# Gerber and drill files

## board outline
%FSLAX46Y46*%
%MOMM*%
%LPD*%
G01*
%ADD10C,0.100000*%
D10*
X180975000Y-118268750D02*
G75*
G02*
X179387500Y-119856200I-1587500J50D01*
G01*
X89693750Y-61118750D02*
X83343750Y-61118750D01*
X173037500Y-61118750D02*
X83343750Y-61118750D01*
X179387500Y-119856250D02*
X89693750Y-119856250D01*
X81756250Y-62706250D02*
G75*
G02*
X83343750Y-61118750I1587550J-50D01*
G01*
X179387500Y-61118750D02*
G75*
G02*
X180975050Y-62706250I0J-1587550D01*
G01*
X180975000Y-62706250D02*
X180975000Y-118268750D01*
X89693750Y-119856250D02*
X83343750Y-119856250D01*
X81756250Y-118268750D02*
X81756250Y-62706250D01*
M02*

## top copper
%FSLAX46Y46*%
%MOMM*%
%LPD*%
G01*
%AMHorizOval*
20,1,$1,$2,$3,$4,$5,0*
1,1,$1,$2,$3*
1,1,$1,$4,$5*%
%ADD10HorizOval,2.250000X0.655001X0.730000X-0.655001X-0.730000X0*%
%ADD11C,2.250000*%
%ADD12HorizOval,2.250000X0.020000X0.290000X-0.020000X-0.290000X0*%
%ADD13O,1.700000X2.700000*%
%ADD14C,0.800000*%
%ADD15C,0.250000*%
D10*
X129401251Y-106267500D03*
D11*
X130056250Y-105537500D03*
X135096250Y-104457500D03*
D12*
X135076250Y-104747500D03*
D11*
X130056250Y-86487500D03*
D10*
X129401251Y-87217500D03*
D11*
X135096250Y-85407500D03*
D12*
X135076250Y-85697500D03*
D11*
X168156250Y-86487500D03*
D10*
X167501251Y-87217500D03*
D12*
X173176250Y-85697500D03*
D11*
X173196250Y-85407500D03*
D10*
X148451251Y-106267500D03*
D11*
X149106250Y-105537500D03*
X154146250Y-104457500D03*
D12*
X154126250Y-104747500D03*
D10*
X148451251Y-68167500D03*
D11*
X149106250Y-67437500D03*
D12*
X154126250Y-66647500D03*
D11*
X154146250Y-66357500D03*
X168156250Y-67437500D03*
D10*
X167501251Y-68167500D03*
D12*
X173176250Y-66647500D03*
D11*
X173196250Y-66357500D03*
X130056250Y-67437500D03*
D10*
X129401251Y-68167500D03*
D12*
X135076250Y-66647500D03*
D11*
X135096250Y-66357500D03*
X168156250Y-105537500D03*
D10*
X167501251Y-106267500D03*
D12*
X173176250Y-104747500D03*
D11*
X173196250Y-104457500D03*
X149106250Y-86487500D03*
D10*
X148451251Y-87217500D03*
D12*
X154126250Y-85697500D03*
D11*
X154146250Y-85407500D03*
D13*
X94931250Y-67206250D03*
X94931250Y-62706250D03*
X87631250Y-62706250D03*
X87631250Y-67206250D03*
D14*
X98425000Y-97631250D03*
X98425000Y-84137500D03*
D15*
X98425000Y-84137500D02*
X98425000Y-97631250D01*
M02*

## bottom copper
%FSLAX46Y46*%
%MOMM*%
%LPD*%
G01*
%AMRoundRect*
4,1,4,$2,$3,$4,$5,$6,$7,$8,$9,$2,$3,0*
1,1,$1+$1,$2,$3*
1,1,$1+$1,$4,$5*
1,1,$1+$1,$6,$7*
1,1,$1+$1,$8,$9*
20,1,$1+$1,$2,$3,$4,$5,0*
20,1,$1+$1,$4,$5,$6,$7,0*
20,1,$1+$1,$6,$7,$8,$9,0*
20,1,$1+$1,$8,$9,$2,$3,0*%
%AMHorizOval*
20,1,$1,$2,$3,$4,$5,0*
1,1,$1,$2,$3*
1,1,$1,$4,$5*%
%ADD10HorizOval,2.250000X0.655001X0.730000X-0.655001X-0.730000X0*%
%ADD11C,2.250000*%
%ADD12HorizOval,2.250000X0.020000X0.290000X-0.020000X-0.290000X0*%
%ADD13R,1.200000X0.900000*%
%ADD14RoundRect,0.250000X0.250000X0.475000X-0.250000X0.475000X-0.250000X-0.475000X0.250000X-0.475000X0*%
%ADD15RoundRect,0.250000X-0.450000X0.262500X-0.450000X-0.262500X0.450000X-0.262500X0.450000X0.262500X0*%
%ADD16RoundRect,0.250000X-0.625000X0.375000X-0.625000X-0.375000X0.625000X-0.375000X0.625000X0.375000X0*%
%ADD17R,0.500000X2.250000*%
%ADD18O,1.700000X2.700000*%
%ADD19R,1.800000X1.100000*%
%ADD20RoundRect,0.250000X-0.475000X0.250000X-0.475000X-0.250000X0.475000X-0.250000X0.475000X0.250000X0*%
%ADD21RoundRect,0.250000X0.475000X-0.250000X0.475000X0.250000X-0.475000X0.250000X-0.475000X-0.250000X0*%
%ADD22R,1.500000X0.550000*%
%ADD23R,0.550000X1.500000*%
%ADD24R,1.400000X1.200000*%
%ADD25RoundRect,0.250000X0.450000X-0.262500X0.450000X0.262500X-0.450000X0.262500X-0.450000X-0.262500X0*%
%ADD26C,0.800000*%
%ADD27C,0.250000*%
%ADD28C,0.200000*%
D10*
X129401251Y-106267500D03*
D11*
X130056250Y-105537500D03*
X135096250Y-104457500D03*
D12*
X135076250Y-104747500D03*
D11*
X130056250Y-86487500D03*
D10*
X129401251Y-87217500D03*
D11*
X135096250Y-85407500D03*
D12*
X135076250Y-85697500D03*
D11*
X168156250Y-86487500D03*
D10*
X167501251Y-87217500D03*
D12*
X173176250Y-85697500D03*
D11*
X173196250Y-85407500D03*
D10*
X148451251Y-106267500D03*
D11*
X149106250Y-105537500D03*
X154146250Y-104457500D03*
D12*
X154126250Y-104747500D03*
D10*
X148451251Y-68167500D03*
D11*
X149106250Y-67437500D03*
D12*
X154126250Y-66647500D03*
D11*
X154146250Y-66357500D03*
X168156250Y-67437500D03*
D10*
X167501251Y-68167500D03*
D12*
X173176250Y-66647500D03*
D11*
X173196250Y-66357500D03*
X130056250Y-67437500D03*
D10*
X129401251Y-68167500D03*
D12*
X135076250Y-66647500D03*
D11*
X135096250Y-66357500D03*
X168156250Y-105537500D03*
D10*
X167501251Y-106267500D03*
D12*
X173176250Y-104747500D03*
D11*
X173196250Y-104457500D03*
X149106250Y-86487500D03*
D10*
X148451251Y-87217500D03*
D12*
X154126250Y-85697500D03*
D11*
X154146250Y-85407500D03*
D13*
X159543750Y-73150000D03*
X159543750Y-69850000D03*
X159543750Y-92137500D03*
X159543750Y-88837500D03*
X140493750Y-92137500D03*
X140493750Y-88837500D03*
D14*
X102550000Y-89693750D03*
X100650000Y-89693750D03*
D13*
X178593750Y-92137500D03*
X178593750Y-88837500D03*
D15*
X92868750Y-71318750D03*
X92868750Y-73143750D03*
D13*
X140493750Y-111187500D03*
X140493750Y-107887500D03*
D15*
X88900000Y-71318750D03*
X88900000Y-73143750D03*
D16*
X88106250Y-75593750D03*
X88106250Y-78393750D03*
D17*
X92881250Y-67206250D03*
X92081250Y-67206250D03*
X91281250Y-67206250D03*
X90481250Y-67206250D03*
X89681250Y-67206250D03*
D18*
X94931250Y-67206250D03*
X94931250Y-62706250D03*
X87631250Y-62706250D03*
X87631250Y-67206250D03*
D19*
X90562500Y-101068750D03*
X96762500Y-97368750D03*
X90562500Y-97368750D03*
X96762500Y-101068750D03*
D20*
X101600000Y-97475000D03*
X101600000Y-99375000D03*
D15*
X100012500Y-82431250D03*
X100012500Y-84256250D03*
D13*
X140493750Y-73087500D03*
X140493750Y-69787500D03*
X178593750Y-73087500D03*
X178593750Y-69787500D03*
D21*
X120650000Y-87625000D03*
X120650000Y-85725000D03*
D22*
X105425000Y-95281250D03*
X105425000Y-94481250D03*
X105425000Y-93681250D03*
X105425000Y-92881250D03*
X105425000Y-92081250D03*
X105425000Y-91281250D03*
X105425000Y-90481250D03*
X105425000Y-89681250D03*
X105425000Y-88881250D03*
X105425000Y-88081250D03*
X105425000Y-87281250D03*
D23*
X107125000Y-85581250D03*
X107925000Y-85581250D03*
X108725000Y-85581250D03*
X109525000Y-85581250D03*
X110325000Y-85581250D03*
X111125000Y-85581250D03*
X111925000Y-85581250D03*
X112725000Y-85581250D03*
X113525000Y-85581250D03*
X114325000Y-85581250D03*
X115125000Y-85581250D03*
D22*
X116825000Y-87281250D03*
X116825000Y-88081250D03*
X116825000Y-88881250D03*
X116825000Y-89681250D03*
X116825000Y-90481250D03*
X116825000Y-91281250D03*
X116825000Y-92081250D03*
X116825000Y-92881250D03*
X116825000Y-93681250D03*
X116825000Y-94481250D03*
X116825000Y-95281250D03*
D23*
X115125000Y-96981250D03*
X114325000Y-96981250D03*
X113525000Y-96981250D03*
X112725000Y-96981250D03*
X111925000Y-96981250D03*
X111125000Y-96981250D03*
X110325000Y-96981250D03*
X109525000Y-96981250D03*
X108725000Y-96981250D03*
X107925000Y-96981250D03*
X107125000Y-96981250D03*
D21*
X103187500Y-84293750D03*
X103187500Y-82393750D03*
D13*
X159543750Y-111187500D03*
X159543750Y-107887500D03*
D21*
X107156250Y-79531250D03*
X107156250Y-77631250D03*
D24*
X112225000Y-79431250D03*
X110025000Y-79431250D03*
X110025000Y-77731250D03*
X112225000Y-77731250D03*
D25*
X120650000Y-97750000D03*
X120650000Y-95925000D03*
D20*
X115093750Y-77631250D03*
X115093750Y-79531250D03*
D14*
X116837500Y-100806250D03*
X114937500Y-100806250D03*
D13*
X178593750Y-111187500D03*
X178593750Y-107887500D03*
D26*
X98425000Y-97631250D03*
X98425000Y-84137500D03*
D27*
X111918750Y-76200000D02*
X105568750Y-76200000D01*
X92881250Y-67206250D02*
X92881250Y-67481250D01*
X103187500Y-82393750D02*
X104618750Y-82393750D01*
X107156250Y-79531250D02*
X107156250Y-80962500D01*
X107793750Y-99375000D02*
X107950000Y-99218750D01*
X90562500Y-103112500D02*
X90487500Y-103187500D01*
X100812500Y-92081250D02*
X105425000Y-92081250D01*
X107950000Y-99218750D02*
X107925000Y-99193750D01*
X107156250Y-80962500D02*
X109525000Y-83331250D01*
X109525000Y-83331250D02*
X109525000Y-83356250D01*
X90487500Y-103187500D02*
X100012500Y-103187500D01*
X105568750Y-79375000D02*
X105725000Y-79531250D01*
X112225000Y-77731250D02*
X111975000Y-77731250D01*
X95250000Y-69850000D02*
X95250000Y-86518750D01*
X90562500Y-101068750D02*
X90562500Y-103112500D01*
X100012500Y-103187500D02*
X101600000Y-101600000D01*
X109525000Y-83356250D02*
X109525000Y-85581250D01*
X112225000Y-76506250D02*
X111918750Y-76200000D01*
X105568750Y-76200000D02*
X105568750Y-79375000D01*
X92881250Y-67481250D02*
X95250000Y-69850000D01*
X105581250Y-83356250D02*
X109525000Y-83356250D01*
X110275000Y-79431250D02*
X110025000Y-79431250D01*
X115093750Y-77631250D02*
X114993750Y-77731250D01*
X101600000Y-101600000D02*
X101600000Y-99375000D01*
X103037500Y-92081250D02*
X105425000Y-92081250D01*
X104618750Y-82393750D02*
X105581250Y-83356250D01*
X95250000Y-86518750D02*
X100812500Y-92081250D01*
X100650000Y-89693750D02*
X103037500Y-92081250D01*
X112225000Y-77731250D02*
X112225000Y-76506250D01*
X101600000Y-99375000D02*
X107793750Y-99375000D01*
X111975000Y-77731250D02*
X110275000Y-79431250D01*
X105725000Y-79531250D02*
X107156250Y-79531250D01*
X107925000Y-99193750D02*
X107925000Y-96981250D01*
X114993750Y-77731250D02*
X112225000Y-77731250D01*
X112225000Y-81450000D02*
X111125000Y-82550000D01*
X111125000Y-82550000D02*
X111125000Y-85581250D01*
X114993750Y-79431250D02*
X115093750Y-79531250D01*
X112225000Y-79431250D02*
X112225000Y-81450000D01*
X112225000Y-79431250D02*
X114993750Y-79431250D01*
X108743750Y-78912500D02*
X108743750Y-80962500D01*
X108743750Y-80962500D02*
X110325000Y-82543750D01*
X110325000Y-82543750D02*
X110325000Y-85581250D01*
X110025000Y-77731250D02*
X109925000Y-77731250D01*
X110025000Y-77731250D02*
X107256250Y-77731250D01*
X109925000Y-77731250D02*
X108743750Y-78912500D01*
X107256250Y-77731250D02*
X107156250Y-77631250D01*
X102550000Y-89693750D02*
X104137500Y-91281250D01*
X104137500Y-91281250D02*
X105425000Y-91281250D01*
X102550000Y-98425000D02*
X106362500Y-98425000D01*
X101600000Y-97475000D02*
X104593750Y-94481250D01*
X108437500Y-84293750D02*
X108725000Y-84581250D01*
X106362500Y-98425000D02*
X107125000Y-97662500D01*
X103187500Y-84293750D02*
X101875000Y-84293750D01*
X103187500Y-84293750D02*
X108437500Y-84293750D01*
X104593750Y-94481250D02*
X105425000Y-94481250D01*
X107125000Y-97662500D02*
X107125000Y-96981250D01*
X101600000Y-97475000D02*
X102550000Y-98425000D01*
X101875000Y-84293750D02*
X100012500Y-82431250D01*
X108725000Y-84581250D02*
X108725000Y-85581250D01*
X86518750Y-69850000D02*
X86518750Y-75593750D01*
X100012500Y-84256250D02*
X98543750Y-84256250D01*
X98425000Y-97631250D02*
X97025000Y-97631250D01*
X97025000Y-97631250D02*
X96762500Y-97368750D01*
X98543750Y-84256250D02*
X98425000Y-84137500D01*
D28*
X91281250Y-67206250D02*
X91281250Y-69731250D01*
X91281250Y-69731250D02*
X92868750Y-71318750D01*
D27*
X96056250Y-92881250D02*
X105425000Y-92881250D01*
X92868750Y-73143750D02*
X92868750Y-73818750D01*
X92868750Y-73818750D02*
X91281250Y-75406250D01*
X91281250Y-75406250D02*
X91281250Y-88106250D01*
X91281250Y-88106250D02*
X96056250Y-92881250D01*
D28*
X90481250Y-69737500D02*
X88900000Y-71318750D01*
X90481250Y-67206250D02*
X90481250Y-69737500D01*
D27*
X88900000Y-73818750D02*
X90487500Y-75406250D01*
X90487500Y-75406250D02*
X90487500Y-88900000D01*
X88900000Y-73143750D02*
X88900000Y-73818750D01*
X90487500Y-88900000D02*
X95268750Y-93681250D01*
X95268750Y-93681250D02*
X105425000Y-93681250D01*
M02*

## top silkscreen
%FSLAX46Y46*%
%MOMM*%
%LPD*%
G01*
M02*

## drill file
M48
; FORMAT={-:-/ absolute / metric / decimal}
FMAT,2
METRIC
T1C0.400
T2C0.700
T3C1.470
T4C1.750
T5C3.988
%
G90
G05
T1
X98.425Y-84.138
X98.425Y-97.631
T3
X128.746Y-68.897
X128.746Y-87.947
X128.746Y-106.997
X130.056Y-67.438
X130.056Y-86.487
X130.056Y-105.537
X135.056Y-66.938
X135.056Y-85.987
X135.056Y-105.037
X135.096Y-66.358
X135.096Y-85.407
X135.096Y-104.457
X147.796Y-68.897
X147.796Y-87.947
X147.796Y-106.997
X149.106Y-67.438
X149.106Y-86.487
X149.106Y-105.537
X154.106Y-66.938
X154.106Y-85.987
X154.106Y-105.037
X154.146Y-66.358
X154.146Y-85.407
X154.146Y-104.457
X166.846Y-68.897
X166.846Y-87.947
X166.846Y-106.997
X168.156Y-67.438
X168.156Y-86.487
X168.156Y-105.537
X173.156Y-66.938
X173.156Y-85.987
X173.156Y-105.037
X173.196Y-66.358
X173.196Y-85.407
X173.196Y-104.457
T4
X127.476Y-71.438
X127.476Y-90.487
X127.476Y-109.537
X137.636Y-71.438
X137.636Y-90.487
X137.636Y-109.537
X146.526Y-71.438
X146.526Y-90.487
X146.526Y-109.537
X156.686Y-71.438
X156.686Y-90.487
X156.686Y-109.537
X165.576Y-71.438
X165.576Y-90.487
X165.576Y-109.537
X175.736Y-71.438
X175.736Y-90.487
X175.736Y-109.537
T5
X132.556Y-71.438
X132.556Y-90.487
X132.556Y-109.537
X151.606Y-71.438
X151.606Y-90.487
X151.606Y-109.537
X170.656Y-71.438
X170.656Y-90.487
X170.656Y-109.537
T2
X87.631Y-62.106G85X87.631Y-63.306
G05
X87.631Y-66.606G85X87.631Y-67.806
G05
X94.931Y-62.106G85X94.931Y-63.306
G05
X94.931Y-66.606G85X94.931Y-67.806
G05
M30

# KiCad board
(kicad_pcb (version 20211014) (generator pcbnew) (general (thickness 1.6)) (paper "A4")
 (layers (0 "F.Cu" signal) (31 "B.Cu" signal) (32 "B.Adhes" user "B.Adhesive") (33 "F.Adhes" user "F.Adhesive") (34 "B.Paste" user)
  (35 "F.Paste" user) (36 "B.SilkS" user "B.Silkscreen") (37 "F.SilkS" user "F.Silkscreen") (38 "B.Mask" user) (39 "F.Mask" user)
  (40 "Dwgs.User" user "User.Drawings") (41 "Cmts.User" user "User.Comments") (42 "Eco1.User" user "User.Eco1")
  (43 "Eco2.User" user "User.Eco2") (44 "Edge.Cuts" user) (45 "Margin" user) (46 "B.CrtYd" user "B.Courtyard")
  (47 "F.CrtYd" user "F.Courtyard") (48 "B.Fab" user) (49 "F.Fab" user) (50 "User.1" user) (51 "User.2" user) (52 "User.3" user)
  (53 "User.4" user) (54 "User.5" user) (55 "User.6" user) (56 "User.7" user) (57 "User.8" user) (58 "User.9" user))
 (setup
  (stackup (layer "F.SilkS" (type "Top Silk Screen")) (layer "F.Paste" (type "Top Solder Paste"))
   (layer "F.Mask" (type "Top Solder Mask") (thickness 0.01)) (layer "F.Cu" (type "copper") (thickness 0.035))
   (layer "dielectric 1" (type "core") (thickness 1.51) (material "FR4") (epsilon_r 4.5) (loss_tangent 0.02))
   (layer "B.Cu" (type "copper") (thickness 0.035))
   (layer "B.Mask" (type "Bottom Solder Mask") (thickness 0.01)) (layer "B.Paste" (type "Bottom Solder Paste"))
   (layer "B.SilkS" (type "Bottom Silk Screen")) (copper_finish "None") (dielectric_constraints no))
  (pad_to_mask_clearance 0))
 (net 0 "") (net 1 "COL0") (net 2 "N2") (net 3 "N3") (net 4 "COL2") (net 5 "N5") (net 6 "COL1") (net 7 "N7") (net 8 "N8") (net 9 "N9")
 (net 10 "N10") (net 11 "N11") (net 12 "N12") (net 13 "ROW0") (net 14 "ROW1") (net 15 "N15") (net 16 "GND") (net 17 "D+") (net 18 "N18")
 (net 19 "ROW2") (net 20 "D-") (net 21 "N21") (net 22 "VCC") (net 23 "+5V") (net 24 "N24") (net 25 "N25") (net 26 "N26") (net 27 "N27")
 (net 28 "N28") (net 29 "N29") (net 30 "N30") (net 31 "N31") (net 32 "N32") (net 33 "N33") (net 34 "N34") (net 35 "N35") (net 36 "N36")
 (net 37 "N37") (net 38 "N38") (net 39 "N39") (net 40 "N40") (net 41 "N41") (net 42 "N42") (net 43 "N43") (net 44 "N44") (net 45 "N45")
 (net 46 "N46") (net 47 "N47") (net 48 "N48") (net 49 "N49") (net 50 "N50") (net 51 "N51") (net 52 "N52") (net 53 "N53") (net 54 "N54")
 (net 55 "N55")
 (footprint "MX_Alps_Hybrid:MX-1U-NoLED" (layer "F.Cu") (at 132.55625 109.5375)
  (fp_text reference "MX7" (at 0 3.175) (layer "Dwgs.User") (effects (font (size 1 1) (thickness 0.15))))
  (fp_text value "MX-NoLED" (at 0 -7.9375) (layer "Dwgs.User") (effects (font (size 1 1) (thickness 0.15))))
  (pad "" np_thru_hole circle locked (at -5.08 0 48.0996) (size 1.75 1.75) (drill 1.75) (layers *.Cu *.Mask))
  (pad "" np_thru_hole circle locked (at 5.08 0 48.0996) (size 1.75 1.75) (drill 1.75) (layers *.Cu *.Mask))
  (pad "" np_thru_hole circle locked (at 0 0) (size 3.9878 3.9878) (drill 3.9878) (layers *.Cu *.Mask))
  (pad "1" thru_hole oval locked (at -3.81 -2.54 48.0996) (size 4.211556 2.25) (drill 1.47 (offset 0.980778 0)) (layers *.Cu "B.Mask")
   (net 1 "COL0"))
  (pad "1" thru_hole circle locked (at -2.5 -4) (size 2.25 2.25) (drill 1.47) (layers *.Cu "B.Mask") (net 1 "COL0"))
  (pad "2" thru_hole circle locked (at 2.54 -5.08) (size 2.25 2.25) (drill 1.47) (layers *.Cu "B.Mask") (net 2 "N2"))
  (pad "2" thru_hole oval locked (at 2.5 -4.5 86.0548) (size 2.831378 2.25) (drill 1.47 (offset 0.290689 0)) (layers *.Cu "B.Mask")
   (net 2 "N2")))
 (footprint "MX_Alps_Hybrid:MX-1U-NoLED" (layer "F.Cu") (at 132.55625 90.4875)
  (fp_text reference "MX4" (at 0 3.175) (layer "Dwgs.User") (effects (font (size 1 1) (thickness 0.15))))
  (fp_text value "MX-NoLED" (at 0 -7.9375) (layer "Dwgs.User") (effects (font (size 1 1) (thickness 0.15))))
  (pad "" np_thru_hole circle locked (at 0 0) (size 3.9878 3.9878) (drill 3.9878) (layers *.Cu *.Mask))
  (pad "" np_thru_hole circle locked (at 5.08 0 48.0996) (size 1.75 1.75) (drill 1.75) (layers *.Cu *.Mask))
  (pad "" np_thru_hole circle locked (at -5.08 0 48.0996) (size 1.75 1.75) (drill 1.75) (layers *.Cu *.Mask))
  (pad "1" thru_hole circle locked (at -2.5 -4) (size 2.25 2.25) (drill 1.47) (layers *.Cu "B.Mask") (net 1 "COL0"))
  (pad "1" thru_hole oval locked (at -3.81 -2.54 48.0996) (size 4.211556 2.25) (drill 1.47 (offset 0.980778 0)) (layers *.Cu "B.Mask")
   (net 1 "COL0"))
  (pad "2" thru_hole circle locked (at 2.54 -5.08) (size 2.25 2.25) (drill 1.47) (layers *.Cu "B.Mask") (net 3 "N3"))
  (pad "2" thru_hole oval locked (at 2.5 -4.5 86.0548) (size 2.831378 2.25) (drill 1.47 (offset 0.290689 0)) (layers *.Cu "B.Mask")
   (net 3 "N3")))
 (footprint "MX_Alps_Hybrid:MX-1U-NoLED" (layer "F.Cu") (at 170.65625 90.4875)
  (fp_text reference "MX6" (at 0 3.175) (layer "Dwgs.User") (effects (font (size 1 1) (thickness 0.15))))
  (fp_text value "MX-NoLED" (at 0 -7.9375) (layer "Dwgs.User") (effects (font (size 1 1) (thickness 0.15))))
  (pad "" np_thru_hole circle locked (at -5.08 0 48.0996) (size 1.75 1.75) (drill 1.75) (layers *.Cu *.Mask))
  (pad "" np_thru_hole circle locked (at 5.08 0 48.0996) (size 1.75 1.75) (drill 1.75) (layers *.Cu *.Mask))
  (pad "" np_thru_hole circle locked (at 0 0) (size 3.9878 3.9878) (drill 3.9878) (layers *.Cu *.Mask))
  (pad "1" thru_hole circle locked (at -2.5 -4) (size 2.25 2.25) (drill 1.47) (layers *.Cu "B.Mask") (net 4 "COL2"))
  (pad "1" thru_hole oval locked (at -3.81 -2.54 48.0996) (size 4.211556 2.25) (drill 1.47 (offset 0.980778 0)) (layers *.Cu "B.Mask")
   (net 4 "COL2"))
  (pad "2" thru_hole oval locked (at 2.5 -4.5 86.0548) (size 2.831378 2.25) (drill 1.47 (offset 0.290689 0)) (layers *.Cu "B.Mask")
   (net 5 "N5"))
  (pad "2" thru_hole circle locked (at 2.54 -5.08) (size 2.25 2.25) (drill 1.47) (layers *.Cu "B.Mask") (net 5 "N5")))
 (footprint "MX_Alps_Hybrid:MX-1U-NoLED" (layer "F.Cu") (at 151.60625 109.5375)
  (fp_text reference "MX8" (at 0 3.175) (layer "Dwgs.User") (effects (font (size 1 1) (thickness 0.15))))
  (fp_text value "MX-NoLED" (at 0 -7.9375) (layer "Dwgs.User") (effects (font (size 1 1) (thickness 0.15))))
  (pad "" np_thru_hole circle locked (at -5.08 0 48.0996) (size 1.75 1.75) (drill 1.75) (layers *.Cu *.Mask))
  (pad "" np_thru_hole circle locked (at 0 0) (size 3.9878 3.9878) (drill 3.9878) (layers *.Cu *.Mask))
  (pad "" np_thru_hole circle locked (at 5.08 0 48.0996) (size 1.75 1.75) (drill 1.75) (layers *.Cu *.Mask))
  (pad "1" thru_hole oval locked (at -3.81 -2.54 48.0996) (size 4.211556 2.25) (drill 1.47 (offset 0.980778 0)) (layers *.Cu "B.Mask")
   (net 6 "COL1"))
  (pad "1" thru_hole circle locked (at -2.5 -4) (size 2.25 2.25) (drill 1.47) (layers *.Cu "B.Mask") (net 6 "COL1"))
  (pad "2" thru_hole circle locked (at 2.54 -5.08) (size 2.25 2.25) (drill 1.47) (layers *.Cu "B.Mask") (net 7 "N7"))
  (pad "2" thru_hole oval locked (at 2.5 -4.5 86.0548) (size 2.831378 2.25) (drill 1.47 (offset 0.290689 0)) (layers *.Cu "B.Mask")
   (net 7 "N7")))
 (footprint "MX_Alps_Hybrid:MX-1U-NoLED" (layer "F.Cu") (at 151.60625 71.4375)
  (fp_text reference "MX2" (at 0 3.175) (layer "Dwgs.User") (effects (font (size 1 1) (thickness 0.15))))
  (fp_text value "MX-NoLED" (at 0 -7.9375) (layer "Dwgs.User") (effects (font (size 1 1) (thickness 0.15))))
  (pad "" np_thru_hole circle locked (at 5.08 0 48.0996) (size 1.75 1.75) (drill 1.75) (layers *.Cu *.Mask))
  (pad "" np_thru_hole circle locked (at -5.08 0 48.0996) (size 1.75 1.75) (drill 1.75) (layers *.Cu *.Mask))
  (pad "" np_thru_hole circle locked (at 0 0) (size 3.9878 3.9878) (drill 3.9878) (layers *.Cu *.Mask))
  (pad "1" thru_hole oval locked (at -3.81 -2.54 48.0996) (size 4.211556 2.25) (drill 1.47 (offset 0.980778 0)) (layers *.Cu "B.Mask")
   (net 6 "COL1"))
  (pad "1" thru_hole circle locked (at -2.5 -4) (size 2.25 2.25) (drill 1.47) (layers *.Cu "B.Mask") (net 6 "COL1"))
  (pad "2" thru_hole oval locked (at 2.5 -4.5 86.0548) (size 2.831378 2.25) (drill 1.47 (offset 0.290689 0)) (layers *.Cu "B.Mask")
   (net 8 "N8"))
  (pad "2" thru_hole circle locked (at 2.54 -5.08) (size 2.25 2.25) (drill 1.47) (layers *.Cu "B.Mask") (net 8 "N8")))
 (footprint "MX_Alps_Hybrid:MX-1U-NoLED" (layer "F.Cu") (at 170.65625 71.4375)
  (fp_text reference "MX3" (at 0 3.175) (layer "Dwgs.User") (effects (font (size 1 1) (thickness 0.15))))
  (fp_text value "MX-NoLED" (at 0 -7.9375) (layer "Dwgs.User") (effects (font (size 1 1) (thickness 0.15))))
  (pad "" np_thru_hole circle locked (at -5.08 0 48.0996) (size 1.75 1.75) (drill 1.75) (layers *.Cu *.Mask))
  (pad "" np_thru_hole circle locked (at 5.08 0 48.0996) (size 1.75 1.75) (drill 1.75) (layers *.Cu *.Mask))
  (pad "" np_thru_hole circle locked (at 0 0) (size 3.9878 3.9878) (drill 3.9878) (layers *.Cu *.Mask))
  (pad "1" thru_hole circle locked (at -2.5 -4) (size 2.25 2.25) (drill 1.47) (layers *.Cu "B.Mask") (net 4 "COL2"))
  (pad "1" thru_hole oval locked (at -3.81 -2.54 48.0996) (size 4.211556 2.25) (drill 1.47 (offset 0.980778 0)) (layers *.Cu "B.Mask")
   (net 4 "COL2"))
  (pad "2" thru_hole oval locked (at 2.5 -4.5 86.0548) (size 2.831378 2.25) (drill 1.47 (offset 0.290689 0)) (layers *.Cu "B.Mask")
   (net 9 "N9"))
  (pad "2" thru_hole circle locked (at 2.54 -5.08) (size 2.25 2.25) (drill 1.47) (layers *.Cu "B.Mask") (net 9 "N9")))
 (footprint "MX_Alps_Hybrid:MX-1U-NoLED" (layer "F.Cu") (at 132.55625 71.4375)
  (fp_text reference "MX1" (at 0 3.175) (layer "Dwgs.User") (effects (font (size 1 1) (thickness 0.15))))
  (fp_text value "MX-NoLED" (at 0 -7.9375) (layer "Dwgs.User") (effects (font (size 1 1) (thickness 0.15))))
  (pad "" np_thru_hole circle locked (at 5.08 0 48.0996) (size 1.75 1.75) (drill 1.75) (layers *.Cu *.Mask))
  (pad "" np_thru_hole circle locked (at -5.08 0 48.0996) (size 1.75 1.75) (drill 1.75) (layers *.Cu *.Mask))
  (pad "" np_thru_hole circle locked (at 0 0) (size 3.9878 3.9878) (drill 3.9878) (layers *.Cu *.Mask))
  (pad "1" thru_hole circle locked (at -2.5 -4) (size 2.25 2.25) (drill 1.47) (layers *.Cu "B.Mask") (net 1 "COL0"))
  (pad "1" thru_hole oval locked (at -3.81 -2.54 48.0996) (size 4.211556 2.25) (drill 1.47 (offset 0.980778 0)) (layers *.Cu "B.Mask")
   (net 1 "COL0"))
  (pad "2" thru_hole oval locked (at 2.5 -4.5 86.0548) (size 2.831378 2.25) (drill 1.47 (offset 0.290689 0)) (layers *.Cu "B.Mask")
   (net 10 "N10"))
  (pad "2" thru_hole circle locked (at 2.54 -5.08) (size 2.25 2.25) (drill 1.47) (layers *.Cu "B.Mask") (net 10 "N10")))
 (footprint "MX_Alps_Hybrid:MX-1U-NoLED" (layer "F.Cu") (at 170.65625 109.5375)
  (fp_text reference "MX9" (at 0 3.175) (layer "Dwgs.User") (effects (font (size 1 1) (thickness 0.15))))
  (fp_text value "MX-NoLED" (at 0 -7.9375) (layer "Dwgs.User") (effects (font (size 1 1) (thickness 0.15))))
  (pad "" np_thru_hole circle locked (at -5.08 0 48.0996) (size 1.75 1.75) (drill 1.75) (layers *.Cu *.Mask))
  (pad "" np_thru_hole circle locked (at 0 0) (size 3.9878 3.9878) (drill 3.9878) (layers *.Cu *.Mask))
  (pad "" np_thru_hole circle locked (at 5.08 0 48.0996) (size 1.75 1.75) (drill 1.75) (layers *.Cu *.Mask))
  (pad "1" thru_hole circle locked (at -2.5 -4) (size 2.25 2.25) (drill 1.47) (layers *.Cu "B.Mask") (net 4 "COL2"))
  (pad "1" thru_hole oval locked (at -3.81 -2.54 48.0996) (size 4.211556 2.25) (drill 1.47 (offset 0.980778 0)) (layers *.Cu "B.Mask")
   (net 4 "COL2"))
  (pad "2" thru_hole oval locked (at 2.5 -4.5 86.0548) (size 2.831378 2.25) (drill 1.47 (offset 0.290689 0)) (layers *.Cu "B.Mask")
   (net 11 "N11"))
  (pad "2" thru_hole circle locked (at 2.54 -5.08) (size 2.25 2.25) (drill 1.47) (layers *.Cu "B.Mask") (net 11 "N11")))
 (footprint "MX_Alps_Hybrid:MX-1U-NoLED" (layer "F.Cu") (at 151.60625 90.4875)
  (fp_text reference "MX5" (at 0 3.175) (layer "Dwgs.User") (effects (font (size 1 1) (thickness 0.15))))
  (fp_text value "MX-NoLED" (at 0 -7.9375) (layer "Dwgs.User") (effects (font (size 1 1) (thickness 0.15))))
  (pad "" np_thru_hole circle locked (at 5.08 0 48.0996) (size 1.75 1.75) (drill 1.75) (layers *.Cu *.Mask))
  (pad "" np_thru_hole circle locked (at -5.08 0 48.0996) (size 1.75 1.75) (drill 1.75) (layers *.Cu *.Mask))
  (pad "" np_thru_hole circle locked (at 0 0) (size 3.9878 3.9878) (drill 3.9878) (layers *.Cu *.Mask))
  (pad "1" thru_hole circle locked (at -2.5 -4) (size 2.25 2.25) (drill 1.47) (layers *.Cu "B.Mask") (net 6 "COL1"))
  (pad "1" thru_hole oval locked (at -3.81 -2.54 48.0996) (size 4.211556 2.25) (drill 1.47 (offset 0.980778 0)) (layers *.Cu "B.Mask")
   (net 6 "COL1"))
  (pad "2" thru_hole oval locked (at 2.5 -4.5 86.0548) (size 2.831378 2.25) (drill 1.47 (offset 0.290689 0)) (layers *.Cu "B.Mask")
   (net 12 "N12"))
  (pad "2" thru_hole circle locked (at 2.54 -5.08) (size 2.25 2.25) (drill 1.47) (layers *.Cu "B.Mask") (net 12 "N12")))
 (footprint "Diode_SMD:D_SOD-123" (layer "B.Cu") (at 159.54375 71.5 90)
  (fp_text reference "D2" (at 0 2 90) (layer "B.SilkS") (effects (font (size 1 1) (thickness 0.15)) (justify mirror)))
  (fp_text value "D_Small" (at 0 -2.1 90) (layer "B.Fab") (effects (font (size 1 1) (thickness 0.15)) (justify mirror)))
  (pad "1" smd rect (at -1.65 0 90) (size 0.9 1.2) (layers "B.Cu" "B.Paste" "B.Mask") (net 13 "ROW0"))
  (pad "2" smd rect (at 1.65 0 90) (size 0.9 1.2) (layers "B.Cu" "B.Paste" "B.Mask") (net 8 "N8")))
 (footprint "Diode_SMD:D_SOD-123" (layer "B.Cu") (at 159.54375 90.4875 90)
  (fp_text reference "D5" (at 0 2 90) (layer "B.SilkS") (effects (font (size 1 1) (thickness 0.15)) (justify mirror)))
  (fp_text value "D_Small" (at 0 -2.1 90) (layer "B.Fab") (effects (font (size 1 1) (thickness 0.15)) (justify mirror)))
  (pad "1" smd rect (at -1.65 0 90) (size 0.9 1.2) (layers "B.Cu" "B.Paste" "B.Mask") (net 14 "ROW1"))
  (pad "2" smd rect (at 1.65 0 90) (size 0.9 1.2) (layers "B.Cu" "B.Paste" "B.Mask") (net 12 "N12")))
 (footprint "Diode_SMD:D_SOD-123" (layer "B.Cu") (at 140.49375 90.4875 90)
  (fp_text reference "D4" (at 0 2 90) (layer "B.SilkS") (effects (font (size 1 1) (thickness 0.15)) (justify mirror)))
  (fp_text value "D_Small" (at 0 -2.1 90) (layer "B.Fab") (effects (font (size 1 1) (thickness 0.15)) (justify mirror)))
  (pad "1" smd rect (at -1.65 0 90) (size 0.9 1.2) (layers "B.Cu" "B.Paste" "B.Mask") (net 14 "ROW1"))
  (pad "2" smd rect (at 1.65 0 90) (size 0.9 1.2) (layers "B.Cu" "B.Paste" "B.Mask") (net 3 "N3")))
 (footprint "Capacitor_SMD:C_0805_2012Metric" (layer "B.Cu") (at 101.6 89.69375 180)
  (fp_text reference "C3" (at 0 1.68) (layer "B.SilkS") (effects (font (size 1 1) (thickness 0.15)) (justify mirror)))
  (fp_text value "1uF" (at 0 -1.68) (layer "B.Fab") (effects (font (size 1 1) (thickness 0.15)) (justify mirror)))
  (pad "1" smd roundrect (at -0.95 0 180) (size 1 1.45) (layers "B.Cu" "B.Paste" "B.Mask") (roundrect_rratio 0.25) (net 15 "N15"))
  (pad "2" smd roundrect (at 0.95 0 180) (size 1 1.45) (layers "B.Cu" "B.Paste" "B.Mask") (roundrect_rratio 0.25) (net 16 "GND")))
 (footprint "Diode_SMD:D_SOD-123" (layer "B.Cu") (at 178.59375 90.4875 90)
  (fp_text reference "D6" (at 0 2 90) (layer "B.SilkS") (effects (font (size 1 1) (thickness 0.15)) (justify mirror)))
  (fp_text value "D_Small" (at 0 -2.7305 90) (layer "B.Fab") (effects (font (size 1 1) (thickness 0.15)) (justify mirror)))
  (pad "1" smd rect (at -1.65 0 90) (size 0.9 1.2) (layers "B.Cu" "B.Paste" "B.Mask") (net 14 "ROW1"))
  (pad "2" smd rect (at 1.65 0 90) (size 0.9 1.2) (layers "B.Cu" "B.Paste" "B.Mask") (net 5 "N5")))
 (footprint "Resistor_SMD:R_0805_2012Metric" (layer "B.Cu") (at 92.86875 72.23125 -90)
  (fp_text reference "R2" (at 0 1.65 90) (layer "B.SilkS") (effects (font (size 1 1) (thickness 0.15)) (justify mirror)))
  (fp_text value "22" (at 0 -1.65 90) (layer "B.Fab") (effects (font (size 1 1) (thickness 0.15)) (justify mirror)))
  (pad "1" smd roundrect (at -0.9125 0 270) (size 1.025 1.4) (layers "B.Cu" "B.Paste" "B.Mask") (roundrect_rratio 0.243902) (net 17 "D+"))
  (pad "2" smd roundrect (at 0.9125 0 270) (size 1.025 1.4) (layers "B.Cu" "B.Paste" "B.Mask") (roundrect_rratio 0.243902) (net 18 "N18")))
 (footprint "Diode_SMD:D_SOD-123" (layer "B.Cu") (at 140.49375 109.5375 90)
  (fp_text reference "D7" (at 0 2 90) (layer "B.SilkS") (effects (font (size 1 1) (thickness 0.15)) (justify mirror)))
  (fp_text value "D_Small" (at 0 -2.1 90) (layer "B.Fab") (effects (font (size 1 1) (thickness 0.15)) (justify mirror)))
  (pad "1" smd rect (at -1.65 0 90) (size 0.9 1.2) (layers "B.Cu" "B.Paste" "B.Mask") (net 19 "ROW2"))
  (pad "2" smd rect (at 1.65 0 90) (size 0.9 1.2) (layers "B.Cu" "B.Paste" "B.Mask") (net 2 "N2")))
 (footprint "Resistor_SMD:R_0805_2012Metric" (layer "B.Cu") (at 88.9 72.23125 -90)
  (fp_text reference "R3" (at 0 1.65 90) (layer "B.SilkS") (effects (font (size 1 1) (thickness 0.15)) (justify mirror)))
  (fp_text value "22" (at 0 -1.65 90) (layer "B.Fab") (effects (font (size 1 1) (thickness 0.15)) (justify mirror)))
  (pad "1" smd roundrect (at -0.9125 0 270) (size 1.025 1.4) (layers "B.Cu" "B.Paste" "B.Mask") (roundrect_rratio 0.243902) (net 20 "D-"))
  (pad "2" smd roundrect (at 0.9125 0 270) (size 1.025 1.4) (layers "B.Cu" "B.Paste" "B.Mask") (roundrect_rratio 0.243902) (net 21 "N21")))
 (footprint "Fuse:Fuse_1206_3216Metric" (layer "B.Cu") (at 88.10625 76.99375 -90)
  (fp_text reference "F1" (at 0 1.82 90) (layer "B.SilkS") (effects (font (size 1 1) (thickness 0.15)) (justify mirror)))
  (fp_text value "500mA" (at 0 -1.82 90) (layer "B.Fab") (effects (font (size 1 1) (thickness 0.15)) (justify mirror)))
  (pad "1" smd roundrect (at -1.4 0 270) (size 1.25 1.75) (layers "B.Cu" "B.Paste" "B.Mask") (roundrect_rratio 0.2) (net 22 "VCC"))
  (pad "2" smd roundrect (at 1.4 0 270) (size 1.25 1.75) (layers "B.Cu" "B.Paste" "B.Mask") (roundrect_rratio 0.2) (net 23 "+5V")))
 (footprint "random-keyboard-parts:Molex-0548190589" (layer "B.Cu") (at 91.28125 62.70625 -90)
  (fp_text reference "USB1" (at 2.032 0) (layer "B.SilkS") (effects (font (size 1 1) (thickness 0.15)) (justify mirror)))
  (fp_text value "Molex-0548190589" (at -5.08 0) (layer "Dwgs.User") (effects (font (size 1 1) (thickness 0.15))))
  (pad "1" smd rect locked (at 4.5 -1.6 270) (size 2.25 0.5) (layers "B.Cu" "B.Paste" "B.Mask") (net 16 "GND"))
  (pad "2" smd rect locked (at 4.5 -0.8 270) (size 2.25 0.5) (layers "B.Cu" "B.Paste" "B.Mask") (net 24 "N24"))
  (pad "3" smd rect locked (at 4.5 0 270) (size 2.25 0.5) (layers "B.Cu" "B.Paste" "B.Mask") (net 17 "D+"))
  (pad "4" smd rect locked (at 4.5 0.8 270) (size 2.25 0.5) (layers "B.Cu" "B.Paste" "B.Mask") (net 20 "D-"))
  (pad "5" smd rect locked (at 4.5 1.6 270) (size 2.25 0.5) (layers "B.Cu" "B.Paste" "B.Mask") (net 22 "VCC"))
  (pad "6" thru_hole oval locked (at 4.5 -3.65 270) (size 2.7 1.7) (drill oval 1.9 0.7) (layers *.Cu *.Mask) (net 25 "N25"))
  (pad "6" thru_hole oval locked (at 0 -3.65 270) (size 2.7 1.7) (drill oval 1.9 0.7) (layers *.Cu *.Mask) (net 25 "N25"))
  (pad "6" thru_hole oval locked (at 0 3.65 270) (size 2.7 1.7) (drill oval 1.9 0.7) (layers *.Cu *.Mask) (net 25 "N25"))
  (pad "6" thru_hole oval locked (at 4.5 3.65 270) (size 2.7 1.7) (drill oval 1.9 0.7) (layers *.Cu *.Mask) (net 25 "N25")))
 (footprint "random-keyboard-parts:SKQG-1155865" (layer "B.Cu") (at 93.6625 99.21875 180)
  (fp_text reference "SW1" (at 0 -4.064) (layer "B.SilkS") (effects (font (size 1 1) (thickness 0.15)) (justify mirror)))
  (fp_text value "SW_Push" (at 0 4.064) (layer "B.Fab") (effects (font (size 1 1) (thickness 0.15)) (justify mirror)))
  (pad "1" smd rect locked (at 3.1 -1.85 180) (size 1.8 1.1) (layers "B.Cu" "B.Paste" "B.Mask") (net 16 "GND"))
  (pad "2" smd rect locked (at -3.1 1.85 180) (size 1.8 1.1) (layers "B.Cu" "B.Paste" "B.Mask") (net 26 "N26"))
  (pad "3" smd rect locked (at 3.1 1.85 180) (size 1.8 1.1) (layers "B.Cu" "B.Paste" "B.Mask"))
  (pad "4" smd rect locked (at -3.1 -1.85 180) (size 1.8 1.1) (layers "B.Cu" "B.Paste" "B.Mask")))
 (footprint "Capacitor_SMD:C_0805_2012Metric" (layer "B.Cu") (at 101.6 98.425 -90)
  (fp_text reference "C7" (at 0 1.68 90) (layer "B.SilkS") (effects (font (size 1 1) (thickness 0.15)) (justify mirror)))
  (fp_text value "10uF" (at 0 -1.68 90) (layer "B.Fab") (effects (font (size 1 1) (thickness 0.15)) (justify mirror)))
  (pad "1" smd roundrect (at -0.95 0 270) (size 1 1.45) (layers "B.Cu" "B.Paste" "B.Mask") (roundrect_rratio 0.25) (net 23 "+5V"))
  (pad "2" smd roundrect (at 0.95 0 270) (size 1 1.45) (layers "B.Cu" "B.Paste" "B.Mask") (roundrect_rratio 0.25) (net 16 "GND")))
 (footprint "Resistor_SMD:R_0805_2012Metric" (layer "B.Cu") (at 100.0125 83.34375 -90)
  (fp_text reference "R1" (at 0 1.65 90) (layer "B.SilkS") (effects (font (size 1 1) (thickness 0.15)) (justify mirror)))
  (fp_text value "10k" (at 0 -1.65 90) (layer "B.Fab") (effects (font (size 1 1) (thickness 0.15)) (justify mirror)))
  (pad "1" smd roundrect (at -0.9125 0 270) (size 1.025 1.4) (layers "B.Cu" "B.Paste" "B.Mask") (roundrect_rratio 0.243902) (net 23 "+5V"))
  (pad "2" smd roundrect (at 0.9125 0 270) (size 1.025 1.4) (layers "B.Cu" "B.Paste" "B.Mask") (roundrect_rratio 0.243902) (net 26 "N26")))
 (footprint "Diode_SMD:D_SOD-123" (layer "B.Cu") (at 140.49375 71.4375 90)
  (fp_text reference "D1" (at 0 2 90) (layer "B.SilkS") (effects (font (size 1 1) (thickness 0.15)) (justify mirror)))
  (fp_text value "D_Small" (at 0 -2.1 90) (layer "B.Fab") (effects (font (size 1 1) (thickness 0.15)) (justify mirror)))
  (pad "1" smd rect (at -1.65 0 90) (size 0.9 1.2) (layers "B.Cu" "B.Paste" "B.Mask") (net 13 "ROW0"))
  (pad "2" smd rect (at 1.65 0 90) (size 0.9 1.2) (layers "B.Cu" "B.Paste" "B.Mask") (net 10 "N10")))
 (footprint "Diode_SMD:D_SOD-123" (layer "B.Cu") (at 178.59375 71.4375 90)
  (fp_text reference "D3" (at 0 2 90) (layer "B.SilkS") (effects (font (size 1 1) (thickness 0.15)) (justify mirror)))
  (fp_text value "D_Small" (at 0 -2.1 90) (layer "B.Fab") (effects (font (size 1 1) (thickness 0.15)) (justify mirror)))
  (pad "1" smd rect (at -1.65 0 90) (size 0.9 1.2) (layers "B.Cu" "B.Paste" "B.Mask") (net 13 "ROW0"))
  (pad "2" smd rect (at 1.65 0 90) (size 0.9 1.2) (layers "B.Cu" "B.Paste" "B.Mask") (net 9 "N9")))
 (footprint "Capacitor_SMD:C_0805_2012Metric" (layer "B.Cu") (at 120.65 86.675 90)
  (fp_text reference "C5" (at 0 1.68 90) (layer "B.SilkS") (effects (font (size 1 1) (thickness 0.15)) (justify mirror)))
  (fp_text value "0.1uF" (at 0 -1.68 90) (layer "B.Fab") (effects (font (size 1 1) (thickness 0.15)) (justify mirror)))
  (pad "1" smd roundrect (at -0.95 0 90) (size 1 1.45) (layers "B.Cu" "B.Paste" "B.Mask") (roundrect_rratio 0.25) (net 23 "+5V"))
  (pad "2" smd roundrect (at 0.95 0 90) (size 1 1.45) (layers "B.Cu" "B.Paste" "B.Mask") (roundrect_rratio 0.25) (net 16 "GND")))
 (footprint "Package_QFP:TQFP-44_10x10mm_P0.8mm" (layer "B.Cu") (at 111.125 91.28125)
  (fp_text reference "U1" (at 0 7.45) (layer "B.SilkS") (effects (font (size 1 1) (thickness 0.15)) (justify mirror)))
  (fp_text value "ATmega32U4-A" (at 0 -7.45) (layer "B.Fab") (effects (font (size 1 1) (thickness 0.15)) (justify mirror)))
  (pad "1" smd rect (at -5.7 4) (size 1.5 0.55) (layers "B.Cu" "B.Paste" "B.Mask") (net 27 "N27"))
  (pad "2" smd rect (at -5.7 3.2) (size 1.5 0.55) (layers "B.Cu" "B.Paste" "B.Mask") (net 23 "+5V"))
  (pad "3" smd rect (at -5.7 2.4) (size 1.5 0.55) (layers "B.Cu" "B.Paste" "B.Mask") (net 21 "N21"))
  (pad "4" smd rect (at -5.7 1.6) (size 1.5 0.55) (layers "B.Cu" "B.Paste" "B.Mask") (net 18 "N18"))
  (pad "5" smd rect (at -5.7 0.8) (size 1.5 0.55) (layers "B.Cu" "B.Paste" "B.Mask") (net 16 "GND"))
  (pad "6" smd rect (at -5.7 0) (size 1.5 0.55) (layers "B.Cu" "B.Paste" "B.Mask") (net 15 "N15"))
  (pad "7" smd rect (at -5.7 -0.8) (size 1.5 0.55) (layers "B.Cu" "B.Paste" "B.Mask") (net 23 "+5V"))
  (pad "8" smd rect (at -5.7 -1.6) (size 1.5 0.55) (layers "B.Cu" "B.Paste" "B.Mask") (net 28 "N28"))
  (pad "9" smd rect (at -5.7 -2.4) (size 1.5 0.55) (layers "B.Cu" "B.Paste" "B.Mask") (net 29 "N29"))
  (pad "10" smd rect (at -5.7 -3.2) (size 1.5 0.55) (layers "B.Cu" "B.Paste" "B.Mask") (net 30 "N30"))
  (pad "11" smd rect (at -5.7 -4) (size 1.5 0.55) (layers "B.Cu" "B.Paste" "B.Mask") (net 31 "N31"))
  (pad "12" smd rect (at -4 -5.7 270) (size 1.5 0.55) (layers "B.Cu" "B.Paste" "B.Mask") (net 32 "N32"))
  (pad "13" smd rect (at -3.2 -5.7 270) (size 1.5 0.55) (layers "B.Cu" "B.Paste" "B.Mask") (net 26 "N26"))
  (pad "14" smd rect (at -2.4 -5.7 270) (size 1.5 0.55) (layers "B.Cu" "B.Paste" "B.Mask") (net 23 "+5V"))
  (pad "15" smd rect (at -1.6 -5.7 270) (size 1.5 0.55) (layers "B.Cu" "B.Paste" "B.Mask") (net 16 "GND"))
  (pad "16" smd rect (at -0.8 -5.7 270) (size 1.5 0.55) (layers "B.Cu" "B.Paste" "B.Mask") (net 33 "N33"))
  (pad "17" smd rect (at 0 -5.7 270) (size 1.5 0.55) (layers "B.Cu" "B.Paste" "B.Mask") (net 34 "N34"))
  (pad "18" smd rect (at 0.8 -5.7 270) (size 1.5 0.55) (layers "B.Cu" "B.Paste" "B.Mask") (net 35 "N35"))
  (pad "19" smd rect (at 1.6 -5.7 270) (size 1.5 0.55) (layers "B.Cu" "B.Paste" "B.Mask") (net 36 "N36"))
  (pad "20" smd rect (at 2.4 -5.7 270) (size 1.5 0.55) (layers "B.Cu" "B.Paste" "B.Mask") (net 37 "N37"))
  (pad "21" smd rect (at 3.2 -5.7 270) (size 1.5 0.55) (layers "B.Cu" "B.Paste" "B.Mask") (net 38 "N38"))
  (pad "22" smd rect (at 4 -5.7 270) (size 1.5 0.55) (layers "B.Cu" "B.Paste" "B.Mask") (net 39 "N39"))
  (pad "23" smd rect (at 5.7 -4) (size 1.5 0.55) (layers "B.Cu" "B.Paste" "B.Mask") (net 16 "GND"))
  (pad "24" smd rect (at 5.7 -3.2) (size 1.5 0.55) (layers "B.Cu" "B.Paste" "B.Mask") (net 23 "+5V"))
  (pad "25" smd rect (at 5.7 -2.4) (size 1.5 0.55) (layers "B.Cu" "B.Paste" "B.Mask") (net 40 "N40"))
  (pad "26" smd rect (at 5.7 -1.6) (size 1.5 0.55) (layers "B.Cu" "B.Paste" "B.Mask") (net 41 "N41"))
  (pad "27" smd rect (at 5.7 -0.8) (size 1.5 0.55) (layers "B.Cu" "B.Paste" "B.Mask") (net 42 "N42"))
  (pad "28" smd rect (at 5.7 0) (size 1.5 0.55) (layers "B.Cu" "B.Paste" "B.Mask") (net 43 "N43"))
  (pad "29" smd rect (at 5.7 0.8) (size 1.5 0.55) (layers "B.Cu" "B.Paste" "B.Mask") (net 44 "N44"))
  (pad "30" smd rect (at 5.7 1.6) (size 1.5 0.55) (layers "B.Cu" "B.Paste" "B.Mask") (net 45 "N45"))
  (pad "31" smd rect (at 5.7 2.4) (size 1.5 0.55) (layers "B.Cu" "B.Paste" "B.Mask") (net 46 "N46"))
  (pad "32" smd rect (at 5.7 3.2) (size 1.5 0.55) (layers "B.Cu" "B.Paste" "B.Mask") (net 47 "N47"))
  (pad "33" smd rect (at 5.7 4) (size 1.5 0.55) (layers "B.Cu" "B.Paste" "B.Mask") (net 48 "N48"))
  (pad "34" smd rect (at 4 5.7 270) (size 1.5 0.55) (layers "B.Cu" "B.Paste" "B.Mask") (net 23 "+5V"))
  (pad "35" smd rect (at 3.2 5.7 270) (size 1.5 0.55) (layers "B.Cu" "B.Paste" "B.Mask") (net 16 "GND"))
  (pad "36" smd rect (at 2.4 5.7 270) (size 1.5 0.55) (layers "B.Cu" "B.Paste" "B.Mask") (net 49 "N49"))
  (pad "37" smd rect (at 1.6 5.7 270) (size 1.5 0.55) (layers "B.Cu" "B.Paste" "B.Mask") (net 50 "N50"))
  (pad "38" smd rect (at 0.8 5.7 270) (size 1.5 0.55) (layers "B.Cu" "B.Paste" "B.Mask") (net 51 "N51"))
  (pad "39" smd rect (at 0 5.7 270) (size 1.5 0.55) (layers "B.Cu" "B.Paste" "B.Mask") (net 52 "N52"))
  (pad "40" smd rect (at -0.8 5.7 270) (size 1.5 0.55) (layers "B.Cu" "B.Paste" "B.Mask") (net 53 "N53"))
  (pad "41" smd rect (at -1.6 5.7 270) (size 1.5 0.55) (layers "B.Cu" "B.Paste" "B.Mask") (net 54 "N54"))
  (pad "42" smd rect (at -2.4 5.7 270) (size 1.5 0.55) (layers "B.Cu" "B.Paste" "B.Mask") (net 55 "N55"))
  (pad "43" smd rect (at -3.2 5.7 270) (size 1.5 0.55) (layers "B.Cu" "B.Paste" "B.Mask") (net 16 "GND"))
  (pad "44" smd rect (at -4 5.7 270) (size 1.5 0.55) (layers "B.Cu" "B.Paste" "B.Mask") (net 23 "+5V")))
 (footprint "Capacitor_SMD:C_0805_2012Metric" (layer "B.Cu") (at 103.1875 83.34375 90)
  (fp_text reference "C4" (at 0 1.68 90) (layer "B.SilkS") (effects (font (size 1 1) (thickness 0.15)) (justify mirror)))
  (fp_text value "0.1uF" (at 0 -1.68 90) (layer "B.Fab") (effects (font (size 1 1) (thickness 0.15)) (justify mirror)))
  (pad "1" smd roundrect (at -0.95 0 90) (size 1 1.45) (layers "B.Cu" "B.Paste" "B.Mask") (roundrect_rratio 0.25) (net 23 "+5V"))
  (pad "2" smd roundrect (at 0.95 0 90) (size 1 1.45) (layers "B.Cu" "B.Paste" "B.Mask") (roundrect_rratio 0.25) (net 16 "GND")))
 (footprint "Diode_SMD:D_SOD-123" (layer "B.Cu") (at 159.54375 109.5375 90)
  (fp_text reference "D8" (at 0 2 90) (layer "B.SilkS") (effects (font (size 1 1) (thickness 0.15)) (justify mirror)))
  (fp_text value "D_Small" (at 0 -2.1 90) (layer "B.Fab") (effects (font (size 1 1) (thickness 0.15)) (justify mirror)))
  (pad "1" smd rect (at -1.65 0 90) (size 0.9 1.2) (layers "B.Cu" "B.Paste" "B.Mask") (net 19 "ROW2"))
  (pad "2" smd rect (at 1.65 0 90) (size 0.9 1.2) (layers "B.Cu" "B.Paste" "B.Mask") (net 7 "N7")))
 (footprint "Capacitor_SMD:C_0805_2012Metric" (layer "B.Cu") (at 107.15625 78.58125 90)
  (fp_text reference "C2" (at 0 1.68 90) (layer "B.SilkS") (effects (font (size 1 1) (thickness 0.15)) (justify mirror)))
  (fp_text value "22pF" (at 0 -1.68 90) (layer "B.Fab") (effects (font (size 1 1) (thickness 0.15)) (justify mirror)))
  (pad "1" smd roundrect (at -0.95 0 90) (size 1 1.45) (layers "B.Cu" "B.Paste" "B.Mask") (roundrect_rratio 0.25) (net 16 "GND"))
  (pad "2" smd roundrect (at 0.95 0 90) (size 1 1.45) (layers "B.Cu" "B.Paste" "B.Mask") (roundrect_rratio 0.25) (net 33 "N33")))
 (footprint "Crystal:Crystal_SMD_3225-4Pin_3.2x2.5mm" (layer "B.Cu") (at 111.125 78.58125 180)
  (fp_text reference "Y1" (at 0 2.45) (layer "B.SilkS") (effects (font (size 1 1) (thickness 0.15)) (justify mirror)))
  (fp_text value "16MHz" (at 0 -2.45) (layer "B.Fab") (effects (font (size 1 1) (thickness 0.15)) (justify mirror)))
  (pad "1" smd rect (at -1.1 -0.85 180) (size 1.4 1.2) (layers "B.Cu" "B.Paste" "B.Mask") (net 34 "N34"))
  (pad "2" smd rect (at 1.1 -0.85 180) (size 1.4 1.2) (layers "B.Cu" "B.Paste" "B.Mask") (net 16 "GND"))
  (pad "3" smd rect (at 1.1 0.85 180) (size 1.4 1.2) (layers "B.Cu" "B.Paste" "B.Mask") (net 33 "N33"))
  (pad "4" smd rect (at -1.1 0.85 180) (size 1.4 1.2) (layers "B.Cu" "B.Paste" "B.Mask") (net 16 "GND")))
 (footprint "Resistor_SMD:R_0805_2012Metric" (layer "B.Cu") (at 120.65 96.8375 90)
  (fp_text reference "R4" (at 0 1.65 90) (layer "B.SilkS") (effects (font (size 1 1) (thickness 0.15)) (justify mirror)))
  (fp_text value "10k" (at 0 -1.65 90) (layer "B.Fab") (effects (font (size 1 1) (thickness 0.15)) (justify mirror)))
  (pad "1" smd roundrect (at -0.9125 0 90) (size 1.025 1.4) (layers "B.Cu" "B.Paste" "B.Mask") (roundrect_rratio 0.243902) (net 16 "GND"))
  (pad "2" smd roundrect (at 0.9125 0 90) (size 1.025 1.4) (layers "B.Cu" "B.Paste" "B.Mask") (roundrect_rratio 0.243902) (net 48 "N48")))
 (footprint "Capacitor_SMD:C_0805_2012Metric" (layer "B.Cu") (at 115.09375 78.58125 -90)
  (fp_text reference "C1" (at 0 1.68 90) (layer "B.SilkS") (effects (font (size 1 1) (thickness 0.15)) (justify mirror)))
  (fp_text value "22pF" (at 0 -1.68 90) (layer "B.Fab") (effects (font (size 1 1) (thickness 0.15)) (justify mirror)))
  (pad "1" smd roundrect (at -0.95 0 270) (size 1 1.45) (layers "B.Cu" "B.Paste" "B.Mask") (roundrect_rratio 0.25) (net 16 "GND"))
  (pad "2" smd roundrect (at 0.95 0 270) (size 1 1.45) (layers "B.Cu" "B.Paste" "B.Mask") (roundrect_rratio 0.25) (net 34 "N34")))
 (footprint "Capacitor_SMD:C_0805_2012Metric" (layer "B.Cu") (at 115.8875 100.80625 180)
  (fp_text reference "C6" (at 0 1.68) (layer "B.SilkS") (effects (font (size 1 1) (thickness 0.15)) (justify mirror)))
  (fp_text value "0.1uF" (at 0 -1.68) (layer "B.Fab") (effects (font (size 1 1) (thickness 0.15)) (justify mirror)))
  (pad "1" smd roundrect (at -0.95 0 180) (size 1 1.45) (layers "B.Cu" "B.Paste" "B.Mask") (roundrect_rratio 0.25) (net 23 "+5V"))
  (pad "2" smd roundrect (at 0.95 0 180) (size 1 1.45) (layers "B.Cu" "B.Paste" "B.Mask") (roundrect_rratio 0.25) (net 16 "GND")))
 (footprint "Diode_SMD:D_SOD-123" (layer "B.Cu") (at 178.59375 109.5375 90)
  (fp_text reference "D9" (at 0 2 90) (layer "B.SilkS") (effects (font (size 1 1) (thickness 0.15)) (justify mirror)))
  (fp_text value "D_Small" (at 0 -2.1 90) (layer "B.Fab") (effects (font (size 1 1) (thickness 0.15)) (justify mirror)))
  (pad "1" smd rect (at -1.65 0 90) (size 0.9 1.2) (layers "B.Cu" "B.Paste" "B.Mask") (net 19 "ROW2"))
  (pad "2" smd rect (at 1.65 0 90) (size 0.9 1.2) (layers "B.Cu" "B.Paste" "B.Mask") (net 11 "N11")))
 (gr_arc (start 180.975 118.26875) (mid 180.510032 119.391282) (end 179.3875 119.85625) (layer "Edge.Cuts") (width 0.1))
 (gr_line (start 89.69375 61.11875) (end 83.34375 61.11875) (layer "Edge.Cuts") (width 0.1))
 (gr_line (start 173.0375 61.11875) (end 83.34375 61.11875) (layer "Edge.Cuts") (width 0.1))
 (gr_line (start 179.3875 119.85625) (end 89.69375 119.85625) (layer "Edge.Cuts") (width 0.1))
 (gr_arc (start 81.75625 62.70625) (mid 82.221218 61.583718) (end 83.34375 61.11875) (layer "Edge.Cuts") (width 0.1))
 (gr_arc (start 179.3875 61.11875) (mid 180.510032 61.583718) (end 180.975 62.70625) (layer "Edge.Cuts") (width 0.1))
 (gr_line (start 180.975 62.70625) (end 180.975 118.26875) (layer "Edge.Cuts") (width 0.1))
 (gr_line (start 89.69375 119.85625) (end 83.34375 119.85625) (layer "Edge.Cuts") (width 0.1))
 (gr_line (start 81.75625 118.26875) (end 81.75625 62.70625) (layer "Edge.Cuts") (width 0.1))
 (segment (start 111.91875 76.2) (end 105.56875 76.2) (width 0.25) (layer "B.Cu") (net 16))
 (segment (start 92.88125 67.20625) (end 92.88125 67.48125) (width 0.25) (layer "B.Cu") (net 16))
 (segment (start 103.1875 82.39375) (end 104.61875 82.39375) (width 0.25) (layer "B.Cu") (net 16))
 (segment (start 107.15625 79.53125) (end 107.15625 80.9625) (width 0.25) (layer "B.Cu") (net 16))
 (segment (start 107.79375 99.375) (end 107.95 99.21875) (width 0.25) (layer "B.Cu") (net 16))
 (segment (start 90.5625 103.1125) (end 90.4875 103.1875) (width 0.25) (layer "B.Cu") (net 16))
 (segment (start 100.8125 92.08125) (end 105.425 92.08125) (width 0.25) (layer "B.Cu") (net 16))
 (segment (start 107.95 99.21875) (end 107.925 99.19375) (width 0.25) (layer "B.Cu") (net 16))
 (segment (start 107.15625 80.9625) (end 109.525 83.33125) (width 0.25) (layer "B.Cu") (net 16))
 (segment (start 109.525 83.33125) (end 109.525 83.35625) (width 0.25) (layer "B.Cu") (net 16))
 (segment (start 90.4875 103.1875) (end 100.0125 103.1875) (width 0.25) (layer "B.Cu") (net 16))
 (segment (start 105.56875 79.375) (end 105.725 79.53125) (width 0.25) (layer "B.Cu") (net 16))
 (segment (start 112.225 77.73125) (end 111.975 77.73125) (width 0.25) (layer "B.Cu") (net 16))
 (segment (start 95.25 69.85) (end 95.25 86.51875) (width 0.25) (layer "B.Cu") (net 16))
 (segment (start 90.5625 101.06875) (end 90.5625 103.1125) (width 0.25) (layer "B.Cu") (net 16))
 (segment (start 100.0125 103.1875) (end 101.6 101.6) (width 0.25) (layer "B.Cu") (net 16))
 (segment (start 109.525 83.35625) (end 109.525 85.58125) (width 0.25) (layer "B.Cu") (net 16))
 (segment (start 112.225 76.50625) (end 111.91875 76.2) (width 0.25) (layer "B.Cu") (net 16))
 (segment (start 105.56875 76.2) (end 105.56875 79.375) (width 0.25) (layer "B.Cu") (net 16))
 (segment (start 92.88125 67.48125) (end 95.25 69.85) (width 0.25) (layer "B.Cu") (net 16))
 (segment (start 105.58125 83.35625) (end 109.525 83.35625) (width 0.25) (layer "B.Cu") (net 16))
 (segment (start 110.275 79.43125) (end 110.025 79.43125) (width 0.25) (layer "B.Cu") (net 16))
 (segment (start 115.09375 77.63125) (end 114.99375 77.73125) (width 0.25) (layer "B.Cu") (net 16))
 (segment (start 101.6 101.6) (end 101.6 99.375) (width 0.25) (layer "B.Cu") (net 16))
 (segment (start 103.0375 92.08125) (end 105.425 92.08125) (width 0.25) (layer "B.Cu") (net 16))
 (segment (start 104.61875 82.39375) (end 105.58125 83.35625) (width 0.25) (layer "B.Cu") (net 16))
 (segment (start 95.25 86.51875) (end 100.8125 92.08125) (width 0.25) (layer "B.Cu") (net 16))
 (segment (start 100.65 89.69375) (end 103.0375 92.08125) (width 0.25) (layer "B.Cu") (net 16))
 (segment (start 112.225 77.73125) (end 112.225 76.50625) (width 0.25) (layer "B.Cu") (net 16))
 (segment (start 101.6 99.375) (end 107.79375 99.375) (width 0.25) (layer "B.Cu") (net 16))
 (segment (start 111.975 77.73125) (end 110.275 79.43125) (width 0.25) (layer "B.Cu") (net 16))
 (segment (start 105.725 79.53125) (end 107.15625 79.53125) (width 0.25) (layer "B.Cu") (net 16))
 (segment (start 107.925 99.19375) (end 107.925 96.98125) (width 0.25) (layer "B.Cu") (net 16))
 (segment (start 114.99375 77.73125) (end 112.225 77.73125) (width 0.25) (layer "B.Cu") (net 16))
 (segment (start 112.225 81.45) (end 111.125 82.55) (width 0.25) (layer "B.Cu") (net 34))
 (segment (start 111.125 82.55) (end 111.125 85.58125) (width 0.25) (layer "B.Cu") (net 34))
 (segment (start 114.99375 79.43125) (end 115.09375 79.53125) (width 0.25) (layer "B.Cu") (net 34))
 (segment (start 112.225 79.43125) (end 112.225 81.45) (width 0.25) (layer "B.Cu") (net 34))
 (segment (start 112.225 79.43125) (end 114.99375 79.43125) (width 0.25) (layer "B.Cu") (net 34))
 (segment (start 108.74375 78.9125) (end 108.74375 80.9625) (width 0.25) (layer "B.Cu") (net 33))
 (segment (start 108.74375 80.9625) (end 110.325 82.54375) (width 0.25) (layer "B.Cu") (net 33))
 (segment (start 110.325 82.54375) (end 110.325 85.58125) (width 0.25) (layer "B.Cu") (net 33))
 (segment (start 110.025 77.73125) (end 109.925 77.73125) (width 0.25) (layer "B.Cu") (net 33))
 (segment (start 110.025 77.73125) (end 107.25625 77.73125) (width 0.25) (layer "B.Cu") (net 33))
 (segment (start 109.925 77.73125) (end 108.74375 78.9125) (width 0.25) (layer "B.Cu") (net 33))
 (segment (start 107.25625 77.73125) (end 107.15625 77.63125) (width 0.25) (layer "B.Cu") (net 33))
 (segment (start 102.55 89.69375) (end 104.1375 91.28125) (width 0.25) (layer "B.Cu") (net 15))
 (segment (start 104.1375 91.28125) (end 105.425 91.28125) (width 0.25) (layer "B.Cu") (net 15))
 (segment (start 102.55 98.425) (end 106.3625 98.425) (width 0.25) (layer "B.Cu") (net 23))
 (segment (start 101.6 97.475) (end 104.59375 94.48125) (width 0.25) (layer "B.Cu") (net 23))
 (segment (start 108.4375 84.29375) (end 108.725 84.58125) (width 0.25) (layer "B.Cu") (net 23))
 (segment (start 106.3625 98.425) (end 107.125 97.6625) (width 0.25) (layer "B.Cu") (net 23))
 (segment (start 103.1875 84.29375) (end 101.875 84.29375) (width 0.25) (layer "B.Cu") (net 23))
 (segment (start 103.1875 84.29375) (end 108.4375 84.29375) (width 0.25) (layer "B.Cu") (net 23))
 (segment (start 104.59375 94.48125) (end 105.425 94.48125) (width 0.25) (layer "B.Cu") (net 23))
 (segment (start 107.125 97.6625) (end 107.125 96.98125) (width 0.25) (layer "B.Cu") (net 23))
 (segment (start 101.6 97.475) (end 102.55 98.425) (width 0.25) (layer "B.Cu") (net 23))
 (segment (start 101.875 84.29375) (end 100.0125 82.43125) (width 0.25) (layer "B.Cu") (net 23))
 (segment (start 108.725 84.58125) (end 108.725 85.58125) (width 0.25) (layer "B.Cu") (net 23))
 (segment (start 86.51875 69.85) (end 86.51875 75.59375) (width 0.25) (layer "B.Cu") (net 22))
 (segment (start 98.425 84.1375) (end 98.425 97.63125) (width 0.25) (layer "F.Cu") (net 26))
 (via (at 98.425 97.63125) (size 0.8) (drill 0.4) (layers "F.Cu" "B.Cu") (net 26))
 (via (at 98.425 84.1375) (size 0.8) (drill 0.4) (layers "F.Cu" "B.Cu") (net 26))
 (segment (start 100.0125 84.25625) (end 98.54375 84.25625) (width 0.25) (layer "B.Cu") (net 26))
 (segment (start 98.425 97.63125) (end 97.025 97.63125) (width 0.25) (layer "B.Cu") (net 26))
 (segment (start 97.025 97.63125) (end 96.7625 97.36875) (width 0.25) (layer "B.Cu") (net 26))
 (segment (start 98.54375 84.25625) (end 98.425 84.1375) (width 0.25) (layer "B.Cu") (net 26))
 (segment (start 91.28125 67.20625) (end 91.28125 69.73125) (width 0.2) (layer "B.Cu") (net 17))
 (segment (start 91.28125 69.73125) (end 92.86875 71.31875) (width 0.2) (layer "B.Cu") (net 17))
 (segment (start 96.05625 92.88125) (end 105.425 92.88125) (width 0.25) (layer "B.Cu") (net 18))
 (segment (start 92.86875 73.14375) (end 92.86875 73.81875) (width 0.25) (layer "B.Cu") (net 18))
 (segment (start 92.86875 73.81875) (end 91.28125 75.40625) (width 0.25) (layer "B.Cu") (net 18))
 (segment (start 91.28125 75.40625) (end 91.28125 88.10625) (width 0.25) (layer "B.Cu") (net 18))
 (segment (start 91.28125 88.10625) (end 96.05625 92.88125) (width 0.25) (layer "B.Cu") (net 18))
 (segment (start 90.48125 69.7375) (end 88.9 71.31875) (width 0.2) (layer "B.Cu") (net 20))
 (segment (start 90.48125 67.20625) (end 90.48125 69.7375) (width 0.2) (layer "B.Cu") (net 20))
 (segment (start 88.9 73.81875) (end 90.4875 75.40625) (width 0.25) (layer "B.Cu") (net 21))
 (segment (start 90.4875 75.40625) (end 90.4875 88.9) (width 0.25) (layer "B.Cu") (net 21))
 (segment (start 88.9 73.14375) (end 88.9 73.81875) (width 0.25) (layer "B.Cu") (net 21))
 (segment (start 90.4875 88.9) (end 95.26875 93.68125) (width 0.25) (layer "B.Cu") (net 21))
 (segment (start 95.26875 93.68125) (end 105.425 93.68125) (width 0.25) (layer "B.Cu") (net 21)))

